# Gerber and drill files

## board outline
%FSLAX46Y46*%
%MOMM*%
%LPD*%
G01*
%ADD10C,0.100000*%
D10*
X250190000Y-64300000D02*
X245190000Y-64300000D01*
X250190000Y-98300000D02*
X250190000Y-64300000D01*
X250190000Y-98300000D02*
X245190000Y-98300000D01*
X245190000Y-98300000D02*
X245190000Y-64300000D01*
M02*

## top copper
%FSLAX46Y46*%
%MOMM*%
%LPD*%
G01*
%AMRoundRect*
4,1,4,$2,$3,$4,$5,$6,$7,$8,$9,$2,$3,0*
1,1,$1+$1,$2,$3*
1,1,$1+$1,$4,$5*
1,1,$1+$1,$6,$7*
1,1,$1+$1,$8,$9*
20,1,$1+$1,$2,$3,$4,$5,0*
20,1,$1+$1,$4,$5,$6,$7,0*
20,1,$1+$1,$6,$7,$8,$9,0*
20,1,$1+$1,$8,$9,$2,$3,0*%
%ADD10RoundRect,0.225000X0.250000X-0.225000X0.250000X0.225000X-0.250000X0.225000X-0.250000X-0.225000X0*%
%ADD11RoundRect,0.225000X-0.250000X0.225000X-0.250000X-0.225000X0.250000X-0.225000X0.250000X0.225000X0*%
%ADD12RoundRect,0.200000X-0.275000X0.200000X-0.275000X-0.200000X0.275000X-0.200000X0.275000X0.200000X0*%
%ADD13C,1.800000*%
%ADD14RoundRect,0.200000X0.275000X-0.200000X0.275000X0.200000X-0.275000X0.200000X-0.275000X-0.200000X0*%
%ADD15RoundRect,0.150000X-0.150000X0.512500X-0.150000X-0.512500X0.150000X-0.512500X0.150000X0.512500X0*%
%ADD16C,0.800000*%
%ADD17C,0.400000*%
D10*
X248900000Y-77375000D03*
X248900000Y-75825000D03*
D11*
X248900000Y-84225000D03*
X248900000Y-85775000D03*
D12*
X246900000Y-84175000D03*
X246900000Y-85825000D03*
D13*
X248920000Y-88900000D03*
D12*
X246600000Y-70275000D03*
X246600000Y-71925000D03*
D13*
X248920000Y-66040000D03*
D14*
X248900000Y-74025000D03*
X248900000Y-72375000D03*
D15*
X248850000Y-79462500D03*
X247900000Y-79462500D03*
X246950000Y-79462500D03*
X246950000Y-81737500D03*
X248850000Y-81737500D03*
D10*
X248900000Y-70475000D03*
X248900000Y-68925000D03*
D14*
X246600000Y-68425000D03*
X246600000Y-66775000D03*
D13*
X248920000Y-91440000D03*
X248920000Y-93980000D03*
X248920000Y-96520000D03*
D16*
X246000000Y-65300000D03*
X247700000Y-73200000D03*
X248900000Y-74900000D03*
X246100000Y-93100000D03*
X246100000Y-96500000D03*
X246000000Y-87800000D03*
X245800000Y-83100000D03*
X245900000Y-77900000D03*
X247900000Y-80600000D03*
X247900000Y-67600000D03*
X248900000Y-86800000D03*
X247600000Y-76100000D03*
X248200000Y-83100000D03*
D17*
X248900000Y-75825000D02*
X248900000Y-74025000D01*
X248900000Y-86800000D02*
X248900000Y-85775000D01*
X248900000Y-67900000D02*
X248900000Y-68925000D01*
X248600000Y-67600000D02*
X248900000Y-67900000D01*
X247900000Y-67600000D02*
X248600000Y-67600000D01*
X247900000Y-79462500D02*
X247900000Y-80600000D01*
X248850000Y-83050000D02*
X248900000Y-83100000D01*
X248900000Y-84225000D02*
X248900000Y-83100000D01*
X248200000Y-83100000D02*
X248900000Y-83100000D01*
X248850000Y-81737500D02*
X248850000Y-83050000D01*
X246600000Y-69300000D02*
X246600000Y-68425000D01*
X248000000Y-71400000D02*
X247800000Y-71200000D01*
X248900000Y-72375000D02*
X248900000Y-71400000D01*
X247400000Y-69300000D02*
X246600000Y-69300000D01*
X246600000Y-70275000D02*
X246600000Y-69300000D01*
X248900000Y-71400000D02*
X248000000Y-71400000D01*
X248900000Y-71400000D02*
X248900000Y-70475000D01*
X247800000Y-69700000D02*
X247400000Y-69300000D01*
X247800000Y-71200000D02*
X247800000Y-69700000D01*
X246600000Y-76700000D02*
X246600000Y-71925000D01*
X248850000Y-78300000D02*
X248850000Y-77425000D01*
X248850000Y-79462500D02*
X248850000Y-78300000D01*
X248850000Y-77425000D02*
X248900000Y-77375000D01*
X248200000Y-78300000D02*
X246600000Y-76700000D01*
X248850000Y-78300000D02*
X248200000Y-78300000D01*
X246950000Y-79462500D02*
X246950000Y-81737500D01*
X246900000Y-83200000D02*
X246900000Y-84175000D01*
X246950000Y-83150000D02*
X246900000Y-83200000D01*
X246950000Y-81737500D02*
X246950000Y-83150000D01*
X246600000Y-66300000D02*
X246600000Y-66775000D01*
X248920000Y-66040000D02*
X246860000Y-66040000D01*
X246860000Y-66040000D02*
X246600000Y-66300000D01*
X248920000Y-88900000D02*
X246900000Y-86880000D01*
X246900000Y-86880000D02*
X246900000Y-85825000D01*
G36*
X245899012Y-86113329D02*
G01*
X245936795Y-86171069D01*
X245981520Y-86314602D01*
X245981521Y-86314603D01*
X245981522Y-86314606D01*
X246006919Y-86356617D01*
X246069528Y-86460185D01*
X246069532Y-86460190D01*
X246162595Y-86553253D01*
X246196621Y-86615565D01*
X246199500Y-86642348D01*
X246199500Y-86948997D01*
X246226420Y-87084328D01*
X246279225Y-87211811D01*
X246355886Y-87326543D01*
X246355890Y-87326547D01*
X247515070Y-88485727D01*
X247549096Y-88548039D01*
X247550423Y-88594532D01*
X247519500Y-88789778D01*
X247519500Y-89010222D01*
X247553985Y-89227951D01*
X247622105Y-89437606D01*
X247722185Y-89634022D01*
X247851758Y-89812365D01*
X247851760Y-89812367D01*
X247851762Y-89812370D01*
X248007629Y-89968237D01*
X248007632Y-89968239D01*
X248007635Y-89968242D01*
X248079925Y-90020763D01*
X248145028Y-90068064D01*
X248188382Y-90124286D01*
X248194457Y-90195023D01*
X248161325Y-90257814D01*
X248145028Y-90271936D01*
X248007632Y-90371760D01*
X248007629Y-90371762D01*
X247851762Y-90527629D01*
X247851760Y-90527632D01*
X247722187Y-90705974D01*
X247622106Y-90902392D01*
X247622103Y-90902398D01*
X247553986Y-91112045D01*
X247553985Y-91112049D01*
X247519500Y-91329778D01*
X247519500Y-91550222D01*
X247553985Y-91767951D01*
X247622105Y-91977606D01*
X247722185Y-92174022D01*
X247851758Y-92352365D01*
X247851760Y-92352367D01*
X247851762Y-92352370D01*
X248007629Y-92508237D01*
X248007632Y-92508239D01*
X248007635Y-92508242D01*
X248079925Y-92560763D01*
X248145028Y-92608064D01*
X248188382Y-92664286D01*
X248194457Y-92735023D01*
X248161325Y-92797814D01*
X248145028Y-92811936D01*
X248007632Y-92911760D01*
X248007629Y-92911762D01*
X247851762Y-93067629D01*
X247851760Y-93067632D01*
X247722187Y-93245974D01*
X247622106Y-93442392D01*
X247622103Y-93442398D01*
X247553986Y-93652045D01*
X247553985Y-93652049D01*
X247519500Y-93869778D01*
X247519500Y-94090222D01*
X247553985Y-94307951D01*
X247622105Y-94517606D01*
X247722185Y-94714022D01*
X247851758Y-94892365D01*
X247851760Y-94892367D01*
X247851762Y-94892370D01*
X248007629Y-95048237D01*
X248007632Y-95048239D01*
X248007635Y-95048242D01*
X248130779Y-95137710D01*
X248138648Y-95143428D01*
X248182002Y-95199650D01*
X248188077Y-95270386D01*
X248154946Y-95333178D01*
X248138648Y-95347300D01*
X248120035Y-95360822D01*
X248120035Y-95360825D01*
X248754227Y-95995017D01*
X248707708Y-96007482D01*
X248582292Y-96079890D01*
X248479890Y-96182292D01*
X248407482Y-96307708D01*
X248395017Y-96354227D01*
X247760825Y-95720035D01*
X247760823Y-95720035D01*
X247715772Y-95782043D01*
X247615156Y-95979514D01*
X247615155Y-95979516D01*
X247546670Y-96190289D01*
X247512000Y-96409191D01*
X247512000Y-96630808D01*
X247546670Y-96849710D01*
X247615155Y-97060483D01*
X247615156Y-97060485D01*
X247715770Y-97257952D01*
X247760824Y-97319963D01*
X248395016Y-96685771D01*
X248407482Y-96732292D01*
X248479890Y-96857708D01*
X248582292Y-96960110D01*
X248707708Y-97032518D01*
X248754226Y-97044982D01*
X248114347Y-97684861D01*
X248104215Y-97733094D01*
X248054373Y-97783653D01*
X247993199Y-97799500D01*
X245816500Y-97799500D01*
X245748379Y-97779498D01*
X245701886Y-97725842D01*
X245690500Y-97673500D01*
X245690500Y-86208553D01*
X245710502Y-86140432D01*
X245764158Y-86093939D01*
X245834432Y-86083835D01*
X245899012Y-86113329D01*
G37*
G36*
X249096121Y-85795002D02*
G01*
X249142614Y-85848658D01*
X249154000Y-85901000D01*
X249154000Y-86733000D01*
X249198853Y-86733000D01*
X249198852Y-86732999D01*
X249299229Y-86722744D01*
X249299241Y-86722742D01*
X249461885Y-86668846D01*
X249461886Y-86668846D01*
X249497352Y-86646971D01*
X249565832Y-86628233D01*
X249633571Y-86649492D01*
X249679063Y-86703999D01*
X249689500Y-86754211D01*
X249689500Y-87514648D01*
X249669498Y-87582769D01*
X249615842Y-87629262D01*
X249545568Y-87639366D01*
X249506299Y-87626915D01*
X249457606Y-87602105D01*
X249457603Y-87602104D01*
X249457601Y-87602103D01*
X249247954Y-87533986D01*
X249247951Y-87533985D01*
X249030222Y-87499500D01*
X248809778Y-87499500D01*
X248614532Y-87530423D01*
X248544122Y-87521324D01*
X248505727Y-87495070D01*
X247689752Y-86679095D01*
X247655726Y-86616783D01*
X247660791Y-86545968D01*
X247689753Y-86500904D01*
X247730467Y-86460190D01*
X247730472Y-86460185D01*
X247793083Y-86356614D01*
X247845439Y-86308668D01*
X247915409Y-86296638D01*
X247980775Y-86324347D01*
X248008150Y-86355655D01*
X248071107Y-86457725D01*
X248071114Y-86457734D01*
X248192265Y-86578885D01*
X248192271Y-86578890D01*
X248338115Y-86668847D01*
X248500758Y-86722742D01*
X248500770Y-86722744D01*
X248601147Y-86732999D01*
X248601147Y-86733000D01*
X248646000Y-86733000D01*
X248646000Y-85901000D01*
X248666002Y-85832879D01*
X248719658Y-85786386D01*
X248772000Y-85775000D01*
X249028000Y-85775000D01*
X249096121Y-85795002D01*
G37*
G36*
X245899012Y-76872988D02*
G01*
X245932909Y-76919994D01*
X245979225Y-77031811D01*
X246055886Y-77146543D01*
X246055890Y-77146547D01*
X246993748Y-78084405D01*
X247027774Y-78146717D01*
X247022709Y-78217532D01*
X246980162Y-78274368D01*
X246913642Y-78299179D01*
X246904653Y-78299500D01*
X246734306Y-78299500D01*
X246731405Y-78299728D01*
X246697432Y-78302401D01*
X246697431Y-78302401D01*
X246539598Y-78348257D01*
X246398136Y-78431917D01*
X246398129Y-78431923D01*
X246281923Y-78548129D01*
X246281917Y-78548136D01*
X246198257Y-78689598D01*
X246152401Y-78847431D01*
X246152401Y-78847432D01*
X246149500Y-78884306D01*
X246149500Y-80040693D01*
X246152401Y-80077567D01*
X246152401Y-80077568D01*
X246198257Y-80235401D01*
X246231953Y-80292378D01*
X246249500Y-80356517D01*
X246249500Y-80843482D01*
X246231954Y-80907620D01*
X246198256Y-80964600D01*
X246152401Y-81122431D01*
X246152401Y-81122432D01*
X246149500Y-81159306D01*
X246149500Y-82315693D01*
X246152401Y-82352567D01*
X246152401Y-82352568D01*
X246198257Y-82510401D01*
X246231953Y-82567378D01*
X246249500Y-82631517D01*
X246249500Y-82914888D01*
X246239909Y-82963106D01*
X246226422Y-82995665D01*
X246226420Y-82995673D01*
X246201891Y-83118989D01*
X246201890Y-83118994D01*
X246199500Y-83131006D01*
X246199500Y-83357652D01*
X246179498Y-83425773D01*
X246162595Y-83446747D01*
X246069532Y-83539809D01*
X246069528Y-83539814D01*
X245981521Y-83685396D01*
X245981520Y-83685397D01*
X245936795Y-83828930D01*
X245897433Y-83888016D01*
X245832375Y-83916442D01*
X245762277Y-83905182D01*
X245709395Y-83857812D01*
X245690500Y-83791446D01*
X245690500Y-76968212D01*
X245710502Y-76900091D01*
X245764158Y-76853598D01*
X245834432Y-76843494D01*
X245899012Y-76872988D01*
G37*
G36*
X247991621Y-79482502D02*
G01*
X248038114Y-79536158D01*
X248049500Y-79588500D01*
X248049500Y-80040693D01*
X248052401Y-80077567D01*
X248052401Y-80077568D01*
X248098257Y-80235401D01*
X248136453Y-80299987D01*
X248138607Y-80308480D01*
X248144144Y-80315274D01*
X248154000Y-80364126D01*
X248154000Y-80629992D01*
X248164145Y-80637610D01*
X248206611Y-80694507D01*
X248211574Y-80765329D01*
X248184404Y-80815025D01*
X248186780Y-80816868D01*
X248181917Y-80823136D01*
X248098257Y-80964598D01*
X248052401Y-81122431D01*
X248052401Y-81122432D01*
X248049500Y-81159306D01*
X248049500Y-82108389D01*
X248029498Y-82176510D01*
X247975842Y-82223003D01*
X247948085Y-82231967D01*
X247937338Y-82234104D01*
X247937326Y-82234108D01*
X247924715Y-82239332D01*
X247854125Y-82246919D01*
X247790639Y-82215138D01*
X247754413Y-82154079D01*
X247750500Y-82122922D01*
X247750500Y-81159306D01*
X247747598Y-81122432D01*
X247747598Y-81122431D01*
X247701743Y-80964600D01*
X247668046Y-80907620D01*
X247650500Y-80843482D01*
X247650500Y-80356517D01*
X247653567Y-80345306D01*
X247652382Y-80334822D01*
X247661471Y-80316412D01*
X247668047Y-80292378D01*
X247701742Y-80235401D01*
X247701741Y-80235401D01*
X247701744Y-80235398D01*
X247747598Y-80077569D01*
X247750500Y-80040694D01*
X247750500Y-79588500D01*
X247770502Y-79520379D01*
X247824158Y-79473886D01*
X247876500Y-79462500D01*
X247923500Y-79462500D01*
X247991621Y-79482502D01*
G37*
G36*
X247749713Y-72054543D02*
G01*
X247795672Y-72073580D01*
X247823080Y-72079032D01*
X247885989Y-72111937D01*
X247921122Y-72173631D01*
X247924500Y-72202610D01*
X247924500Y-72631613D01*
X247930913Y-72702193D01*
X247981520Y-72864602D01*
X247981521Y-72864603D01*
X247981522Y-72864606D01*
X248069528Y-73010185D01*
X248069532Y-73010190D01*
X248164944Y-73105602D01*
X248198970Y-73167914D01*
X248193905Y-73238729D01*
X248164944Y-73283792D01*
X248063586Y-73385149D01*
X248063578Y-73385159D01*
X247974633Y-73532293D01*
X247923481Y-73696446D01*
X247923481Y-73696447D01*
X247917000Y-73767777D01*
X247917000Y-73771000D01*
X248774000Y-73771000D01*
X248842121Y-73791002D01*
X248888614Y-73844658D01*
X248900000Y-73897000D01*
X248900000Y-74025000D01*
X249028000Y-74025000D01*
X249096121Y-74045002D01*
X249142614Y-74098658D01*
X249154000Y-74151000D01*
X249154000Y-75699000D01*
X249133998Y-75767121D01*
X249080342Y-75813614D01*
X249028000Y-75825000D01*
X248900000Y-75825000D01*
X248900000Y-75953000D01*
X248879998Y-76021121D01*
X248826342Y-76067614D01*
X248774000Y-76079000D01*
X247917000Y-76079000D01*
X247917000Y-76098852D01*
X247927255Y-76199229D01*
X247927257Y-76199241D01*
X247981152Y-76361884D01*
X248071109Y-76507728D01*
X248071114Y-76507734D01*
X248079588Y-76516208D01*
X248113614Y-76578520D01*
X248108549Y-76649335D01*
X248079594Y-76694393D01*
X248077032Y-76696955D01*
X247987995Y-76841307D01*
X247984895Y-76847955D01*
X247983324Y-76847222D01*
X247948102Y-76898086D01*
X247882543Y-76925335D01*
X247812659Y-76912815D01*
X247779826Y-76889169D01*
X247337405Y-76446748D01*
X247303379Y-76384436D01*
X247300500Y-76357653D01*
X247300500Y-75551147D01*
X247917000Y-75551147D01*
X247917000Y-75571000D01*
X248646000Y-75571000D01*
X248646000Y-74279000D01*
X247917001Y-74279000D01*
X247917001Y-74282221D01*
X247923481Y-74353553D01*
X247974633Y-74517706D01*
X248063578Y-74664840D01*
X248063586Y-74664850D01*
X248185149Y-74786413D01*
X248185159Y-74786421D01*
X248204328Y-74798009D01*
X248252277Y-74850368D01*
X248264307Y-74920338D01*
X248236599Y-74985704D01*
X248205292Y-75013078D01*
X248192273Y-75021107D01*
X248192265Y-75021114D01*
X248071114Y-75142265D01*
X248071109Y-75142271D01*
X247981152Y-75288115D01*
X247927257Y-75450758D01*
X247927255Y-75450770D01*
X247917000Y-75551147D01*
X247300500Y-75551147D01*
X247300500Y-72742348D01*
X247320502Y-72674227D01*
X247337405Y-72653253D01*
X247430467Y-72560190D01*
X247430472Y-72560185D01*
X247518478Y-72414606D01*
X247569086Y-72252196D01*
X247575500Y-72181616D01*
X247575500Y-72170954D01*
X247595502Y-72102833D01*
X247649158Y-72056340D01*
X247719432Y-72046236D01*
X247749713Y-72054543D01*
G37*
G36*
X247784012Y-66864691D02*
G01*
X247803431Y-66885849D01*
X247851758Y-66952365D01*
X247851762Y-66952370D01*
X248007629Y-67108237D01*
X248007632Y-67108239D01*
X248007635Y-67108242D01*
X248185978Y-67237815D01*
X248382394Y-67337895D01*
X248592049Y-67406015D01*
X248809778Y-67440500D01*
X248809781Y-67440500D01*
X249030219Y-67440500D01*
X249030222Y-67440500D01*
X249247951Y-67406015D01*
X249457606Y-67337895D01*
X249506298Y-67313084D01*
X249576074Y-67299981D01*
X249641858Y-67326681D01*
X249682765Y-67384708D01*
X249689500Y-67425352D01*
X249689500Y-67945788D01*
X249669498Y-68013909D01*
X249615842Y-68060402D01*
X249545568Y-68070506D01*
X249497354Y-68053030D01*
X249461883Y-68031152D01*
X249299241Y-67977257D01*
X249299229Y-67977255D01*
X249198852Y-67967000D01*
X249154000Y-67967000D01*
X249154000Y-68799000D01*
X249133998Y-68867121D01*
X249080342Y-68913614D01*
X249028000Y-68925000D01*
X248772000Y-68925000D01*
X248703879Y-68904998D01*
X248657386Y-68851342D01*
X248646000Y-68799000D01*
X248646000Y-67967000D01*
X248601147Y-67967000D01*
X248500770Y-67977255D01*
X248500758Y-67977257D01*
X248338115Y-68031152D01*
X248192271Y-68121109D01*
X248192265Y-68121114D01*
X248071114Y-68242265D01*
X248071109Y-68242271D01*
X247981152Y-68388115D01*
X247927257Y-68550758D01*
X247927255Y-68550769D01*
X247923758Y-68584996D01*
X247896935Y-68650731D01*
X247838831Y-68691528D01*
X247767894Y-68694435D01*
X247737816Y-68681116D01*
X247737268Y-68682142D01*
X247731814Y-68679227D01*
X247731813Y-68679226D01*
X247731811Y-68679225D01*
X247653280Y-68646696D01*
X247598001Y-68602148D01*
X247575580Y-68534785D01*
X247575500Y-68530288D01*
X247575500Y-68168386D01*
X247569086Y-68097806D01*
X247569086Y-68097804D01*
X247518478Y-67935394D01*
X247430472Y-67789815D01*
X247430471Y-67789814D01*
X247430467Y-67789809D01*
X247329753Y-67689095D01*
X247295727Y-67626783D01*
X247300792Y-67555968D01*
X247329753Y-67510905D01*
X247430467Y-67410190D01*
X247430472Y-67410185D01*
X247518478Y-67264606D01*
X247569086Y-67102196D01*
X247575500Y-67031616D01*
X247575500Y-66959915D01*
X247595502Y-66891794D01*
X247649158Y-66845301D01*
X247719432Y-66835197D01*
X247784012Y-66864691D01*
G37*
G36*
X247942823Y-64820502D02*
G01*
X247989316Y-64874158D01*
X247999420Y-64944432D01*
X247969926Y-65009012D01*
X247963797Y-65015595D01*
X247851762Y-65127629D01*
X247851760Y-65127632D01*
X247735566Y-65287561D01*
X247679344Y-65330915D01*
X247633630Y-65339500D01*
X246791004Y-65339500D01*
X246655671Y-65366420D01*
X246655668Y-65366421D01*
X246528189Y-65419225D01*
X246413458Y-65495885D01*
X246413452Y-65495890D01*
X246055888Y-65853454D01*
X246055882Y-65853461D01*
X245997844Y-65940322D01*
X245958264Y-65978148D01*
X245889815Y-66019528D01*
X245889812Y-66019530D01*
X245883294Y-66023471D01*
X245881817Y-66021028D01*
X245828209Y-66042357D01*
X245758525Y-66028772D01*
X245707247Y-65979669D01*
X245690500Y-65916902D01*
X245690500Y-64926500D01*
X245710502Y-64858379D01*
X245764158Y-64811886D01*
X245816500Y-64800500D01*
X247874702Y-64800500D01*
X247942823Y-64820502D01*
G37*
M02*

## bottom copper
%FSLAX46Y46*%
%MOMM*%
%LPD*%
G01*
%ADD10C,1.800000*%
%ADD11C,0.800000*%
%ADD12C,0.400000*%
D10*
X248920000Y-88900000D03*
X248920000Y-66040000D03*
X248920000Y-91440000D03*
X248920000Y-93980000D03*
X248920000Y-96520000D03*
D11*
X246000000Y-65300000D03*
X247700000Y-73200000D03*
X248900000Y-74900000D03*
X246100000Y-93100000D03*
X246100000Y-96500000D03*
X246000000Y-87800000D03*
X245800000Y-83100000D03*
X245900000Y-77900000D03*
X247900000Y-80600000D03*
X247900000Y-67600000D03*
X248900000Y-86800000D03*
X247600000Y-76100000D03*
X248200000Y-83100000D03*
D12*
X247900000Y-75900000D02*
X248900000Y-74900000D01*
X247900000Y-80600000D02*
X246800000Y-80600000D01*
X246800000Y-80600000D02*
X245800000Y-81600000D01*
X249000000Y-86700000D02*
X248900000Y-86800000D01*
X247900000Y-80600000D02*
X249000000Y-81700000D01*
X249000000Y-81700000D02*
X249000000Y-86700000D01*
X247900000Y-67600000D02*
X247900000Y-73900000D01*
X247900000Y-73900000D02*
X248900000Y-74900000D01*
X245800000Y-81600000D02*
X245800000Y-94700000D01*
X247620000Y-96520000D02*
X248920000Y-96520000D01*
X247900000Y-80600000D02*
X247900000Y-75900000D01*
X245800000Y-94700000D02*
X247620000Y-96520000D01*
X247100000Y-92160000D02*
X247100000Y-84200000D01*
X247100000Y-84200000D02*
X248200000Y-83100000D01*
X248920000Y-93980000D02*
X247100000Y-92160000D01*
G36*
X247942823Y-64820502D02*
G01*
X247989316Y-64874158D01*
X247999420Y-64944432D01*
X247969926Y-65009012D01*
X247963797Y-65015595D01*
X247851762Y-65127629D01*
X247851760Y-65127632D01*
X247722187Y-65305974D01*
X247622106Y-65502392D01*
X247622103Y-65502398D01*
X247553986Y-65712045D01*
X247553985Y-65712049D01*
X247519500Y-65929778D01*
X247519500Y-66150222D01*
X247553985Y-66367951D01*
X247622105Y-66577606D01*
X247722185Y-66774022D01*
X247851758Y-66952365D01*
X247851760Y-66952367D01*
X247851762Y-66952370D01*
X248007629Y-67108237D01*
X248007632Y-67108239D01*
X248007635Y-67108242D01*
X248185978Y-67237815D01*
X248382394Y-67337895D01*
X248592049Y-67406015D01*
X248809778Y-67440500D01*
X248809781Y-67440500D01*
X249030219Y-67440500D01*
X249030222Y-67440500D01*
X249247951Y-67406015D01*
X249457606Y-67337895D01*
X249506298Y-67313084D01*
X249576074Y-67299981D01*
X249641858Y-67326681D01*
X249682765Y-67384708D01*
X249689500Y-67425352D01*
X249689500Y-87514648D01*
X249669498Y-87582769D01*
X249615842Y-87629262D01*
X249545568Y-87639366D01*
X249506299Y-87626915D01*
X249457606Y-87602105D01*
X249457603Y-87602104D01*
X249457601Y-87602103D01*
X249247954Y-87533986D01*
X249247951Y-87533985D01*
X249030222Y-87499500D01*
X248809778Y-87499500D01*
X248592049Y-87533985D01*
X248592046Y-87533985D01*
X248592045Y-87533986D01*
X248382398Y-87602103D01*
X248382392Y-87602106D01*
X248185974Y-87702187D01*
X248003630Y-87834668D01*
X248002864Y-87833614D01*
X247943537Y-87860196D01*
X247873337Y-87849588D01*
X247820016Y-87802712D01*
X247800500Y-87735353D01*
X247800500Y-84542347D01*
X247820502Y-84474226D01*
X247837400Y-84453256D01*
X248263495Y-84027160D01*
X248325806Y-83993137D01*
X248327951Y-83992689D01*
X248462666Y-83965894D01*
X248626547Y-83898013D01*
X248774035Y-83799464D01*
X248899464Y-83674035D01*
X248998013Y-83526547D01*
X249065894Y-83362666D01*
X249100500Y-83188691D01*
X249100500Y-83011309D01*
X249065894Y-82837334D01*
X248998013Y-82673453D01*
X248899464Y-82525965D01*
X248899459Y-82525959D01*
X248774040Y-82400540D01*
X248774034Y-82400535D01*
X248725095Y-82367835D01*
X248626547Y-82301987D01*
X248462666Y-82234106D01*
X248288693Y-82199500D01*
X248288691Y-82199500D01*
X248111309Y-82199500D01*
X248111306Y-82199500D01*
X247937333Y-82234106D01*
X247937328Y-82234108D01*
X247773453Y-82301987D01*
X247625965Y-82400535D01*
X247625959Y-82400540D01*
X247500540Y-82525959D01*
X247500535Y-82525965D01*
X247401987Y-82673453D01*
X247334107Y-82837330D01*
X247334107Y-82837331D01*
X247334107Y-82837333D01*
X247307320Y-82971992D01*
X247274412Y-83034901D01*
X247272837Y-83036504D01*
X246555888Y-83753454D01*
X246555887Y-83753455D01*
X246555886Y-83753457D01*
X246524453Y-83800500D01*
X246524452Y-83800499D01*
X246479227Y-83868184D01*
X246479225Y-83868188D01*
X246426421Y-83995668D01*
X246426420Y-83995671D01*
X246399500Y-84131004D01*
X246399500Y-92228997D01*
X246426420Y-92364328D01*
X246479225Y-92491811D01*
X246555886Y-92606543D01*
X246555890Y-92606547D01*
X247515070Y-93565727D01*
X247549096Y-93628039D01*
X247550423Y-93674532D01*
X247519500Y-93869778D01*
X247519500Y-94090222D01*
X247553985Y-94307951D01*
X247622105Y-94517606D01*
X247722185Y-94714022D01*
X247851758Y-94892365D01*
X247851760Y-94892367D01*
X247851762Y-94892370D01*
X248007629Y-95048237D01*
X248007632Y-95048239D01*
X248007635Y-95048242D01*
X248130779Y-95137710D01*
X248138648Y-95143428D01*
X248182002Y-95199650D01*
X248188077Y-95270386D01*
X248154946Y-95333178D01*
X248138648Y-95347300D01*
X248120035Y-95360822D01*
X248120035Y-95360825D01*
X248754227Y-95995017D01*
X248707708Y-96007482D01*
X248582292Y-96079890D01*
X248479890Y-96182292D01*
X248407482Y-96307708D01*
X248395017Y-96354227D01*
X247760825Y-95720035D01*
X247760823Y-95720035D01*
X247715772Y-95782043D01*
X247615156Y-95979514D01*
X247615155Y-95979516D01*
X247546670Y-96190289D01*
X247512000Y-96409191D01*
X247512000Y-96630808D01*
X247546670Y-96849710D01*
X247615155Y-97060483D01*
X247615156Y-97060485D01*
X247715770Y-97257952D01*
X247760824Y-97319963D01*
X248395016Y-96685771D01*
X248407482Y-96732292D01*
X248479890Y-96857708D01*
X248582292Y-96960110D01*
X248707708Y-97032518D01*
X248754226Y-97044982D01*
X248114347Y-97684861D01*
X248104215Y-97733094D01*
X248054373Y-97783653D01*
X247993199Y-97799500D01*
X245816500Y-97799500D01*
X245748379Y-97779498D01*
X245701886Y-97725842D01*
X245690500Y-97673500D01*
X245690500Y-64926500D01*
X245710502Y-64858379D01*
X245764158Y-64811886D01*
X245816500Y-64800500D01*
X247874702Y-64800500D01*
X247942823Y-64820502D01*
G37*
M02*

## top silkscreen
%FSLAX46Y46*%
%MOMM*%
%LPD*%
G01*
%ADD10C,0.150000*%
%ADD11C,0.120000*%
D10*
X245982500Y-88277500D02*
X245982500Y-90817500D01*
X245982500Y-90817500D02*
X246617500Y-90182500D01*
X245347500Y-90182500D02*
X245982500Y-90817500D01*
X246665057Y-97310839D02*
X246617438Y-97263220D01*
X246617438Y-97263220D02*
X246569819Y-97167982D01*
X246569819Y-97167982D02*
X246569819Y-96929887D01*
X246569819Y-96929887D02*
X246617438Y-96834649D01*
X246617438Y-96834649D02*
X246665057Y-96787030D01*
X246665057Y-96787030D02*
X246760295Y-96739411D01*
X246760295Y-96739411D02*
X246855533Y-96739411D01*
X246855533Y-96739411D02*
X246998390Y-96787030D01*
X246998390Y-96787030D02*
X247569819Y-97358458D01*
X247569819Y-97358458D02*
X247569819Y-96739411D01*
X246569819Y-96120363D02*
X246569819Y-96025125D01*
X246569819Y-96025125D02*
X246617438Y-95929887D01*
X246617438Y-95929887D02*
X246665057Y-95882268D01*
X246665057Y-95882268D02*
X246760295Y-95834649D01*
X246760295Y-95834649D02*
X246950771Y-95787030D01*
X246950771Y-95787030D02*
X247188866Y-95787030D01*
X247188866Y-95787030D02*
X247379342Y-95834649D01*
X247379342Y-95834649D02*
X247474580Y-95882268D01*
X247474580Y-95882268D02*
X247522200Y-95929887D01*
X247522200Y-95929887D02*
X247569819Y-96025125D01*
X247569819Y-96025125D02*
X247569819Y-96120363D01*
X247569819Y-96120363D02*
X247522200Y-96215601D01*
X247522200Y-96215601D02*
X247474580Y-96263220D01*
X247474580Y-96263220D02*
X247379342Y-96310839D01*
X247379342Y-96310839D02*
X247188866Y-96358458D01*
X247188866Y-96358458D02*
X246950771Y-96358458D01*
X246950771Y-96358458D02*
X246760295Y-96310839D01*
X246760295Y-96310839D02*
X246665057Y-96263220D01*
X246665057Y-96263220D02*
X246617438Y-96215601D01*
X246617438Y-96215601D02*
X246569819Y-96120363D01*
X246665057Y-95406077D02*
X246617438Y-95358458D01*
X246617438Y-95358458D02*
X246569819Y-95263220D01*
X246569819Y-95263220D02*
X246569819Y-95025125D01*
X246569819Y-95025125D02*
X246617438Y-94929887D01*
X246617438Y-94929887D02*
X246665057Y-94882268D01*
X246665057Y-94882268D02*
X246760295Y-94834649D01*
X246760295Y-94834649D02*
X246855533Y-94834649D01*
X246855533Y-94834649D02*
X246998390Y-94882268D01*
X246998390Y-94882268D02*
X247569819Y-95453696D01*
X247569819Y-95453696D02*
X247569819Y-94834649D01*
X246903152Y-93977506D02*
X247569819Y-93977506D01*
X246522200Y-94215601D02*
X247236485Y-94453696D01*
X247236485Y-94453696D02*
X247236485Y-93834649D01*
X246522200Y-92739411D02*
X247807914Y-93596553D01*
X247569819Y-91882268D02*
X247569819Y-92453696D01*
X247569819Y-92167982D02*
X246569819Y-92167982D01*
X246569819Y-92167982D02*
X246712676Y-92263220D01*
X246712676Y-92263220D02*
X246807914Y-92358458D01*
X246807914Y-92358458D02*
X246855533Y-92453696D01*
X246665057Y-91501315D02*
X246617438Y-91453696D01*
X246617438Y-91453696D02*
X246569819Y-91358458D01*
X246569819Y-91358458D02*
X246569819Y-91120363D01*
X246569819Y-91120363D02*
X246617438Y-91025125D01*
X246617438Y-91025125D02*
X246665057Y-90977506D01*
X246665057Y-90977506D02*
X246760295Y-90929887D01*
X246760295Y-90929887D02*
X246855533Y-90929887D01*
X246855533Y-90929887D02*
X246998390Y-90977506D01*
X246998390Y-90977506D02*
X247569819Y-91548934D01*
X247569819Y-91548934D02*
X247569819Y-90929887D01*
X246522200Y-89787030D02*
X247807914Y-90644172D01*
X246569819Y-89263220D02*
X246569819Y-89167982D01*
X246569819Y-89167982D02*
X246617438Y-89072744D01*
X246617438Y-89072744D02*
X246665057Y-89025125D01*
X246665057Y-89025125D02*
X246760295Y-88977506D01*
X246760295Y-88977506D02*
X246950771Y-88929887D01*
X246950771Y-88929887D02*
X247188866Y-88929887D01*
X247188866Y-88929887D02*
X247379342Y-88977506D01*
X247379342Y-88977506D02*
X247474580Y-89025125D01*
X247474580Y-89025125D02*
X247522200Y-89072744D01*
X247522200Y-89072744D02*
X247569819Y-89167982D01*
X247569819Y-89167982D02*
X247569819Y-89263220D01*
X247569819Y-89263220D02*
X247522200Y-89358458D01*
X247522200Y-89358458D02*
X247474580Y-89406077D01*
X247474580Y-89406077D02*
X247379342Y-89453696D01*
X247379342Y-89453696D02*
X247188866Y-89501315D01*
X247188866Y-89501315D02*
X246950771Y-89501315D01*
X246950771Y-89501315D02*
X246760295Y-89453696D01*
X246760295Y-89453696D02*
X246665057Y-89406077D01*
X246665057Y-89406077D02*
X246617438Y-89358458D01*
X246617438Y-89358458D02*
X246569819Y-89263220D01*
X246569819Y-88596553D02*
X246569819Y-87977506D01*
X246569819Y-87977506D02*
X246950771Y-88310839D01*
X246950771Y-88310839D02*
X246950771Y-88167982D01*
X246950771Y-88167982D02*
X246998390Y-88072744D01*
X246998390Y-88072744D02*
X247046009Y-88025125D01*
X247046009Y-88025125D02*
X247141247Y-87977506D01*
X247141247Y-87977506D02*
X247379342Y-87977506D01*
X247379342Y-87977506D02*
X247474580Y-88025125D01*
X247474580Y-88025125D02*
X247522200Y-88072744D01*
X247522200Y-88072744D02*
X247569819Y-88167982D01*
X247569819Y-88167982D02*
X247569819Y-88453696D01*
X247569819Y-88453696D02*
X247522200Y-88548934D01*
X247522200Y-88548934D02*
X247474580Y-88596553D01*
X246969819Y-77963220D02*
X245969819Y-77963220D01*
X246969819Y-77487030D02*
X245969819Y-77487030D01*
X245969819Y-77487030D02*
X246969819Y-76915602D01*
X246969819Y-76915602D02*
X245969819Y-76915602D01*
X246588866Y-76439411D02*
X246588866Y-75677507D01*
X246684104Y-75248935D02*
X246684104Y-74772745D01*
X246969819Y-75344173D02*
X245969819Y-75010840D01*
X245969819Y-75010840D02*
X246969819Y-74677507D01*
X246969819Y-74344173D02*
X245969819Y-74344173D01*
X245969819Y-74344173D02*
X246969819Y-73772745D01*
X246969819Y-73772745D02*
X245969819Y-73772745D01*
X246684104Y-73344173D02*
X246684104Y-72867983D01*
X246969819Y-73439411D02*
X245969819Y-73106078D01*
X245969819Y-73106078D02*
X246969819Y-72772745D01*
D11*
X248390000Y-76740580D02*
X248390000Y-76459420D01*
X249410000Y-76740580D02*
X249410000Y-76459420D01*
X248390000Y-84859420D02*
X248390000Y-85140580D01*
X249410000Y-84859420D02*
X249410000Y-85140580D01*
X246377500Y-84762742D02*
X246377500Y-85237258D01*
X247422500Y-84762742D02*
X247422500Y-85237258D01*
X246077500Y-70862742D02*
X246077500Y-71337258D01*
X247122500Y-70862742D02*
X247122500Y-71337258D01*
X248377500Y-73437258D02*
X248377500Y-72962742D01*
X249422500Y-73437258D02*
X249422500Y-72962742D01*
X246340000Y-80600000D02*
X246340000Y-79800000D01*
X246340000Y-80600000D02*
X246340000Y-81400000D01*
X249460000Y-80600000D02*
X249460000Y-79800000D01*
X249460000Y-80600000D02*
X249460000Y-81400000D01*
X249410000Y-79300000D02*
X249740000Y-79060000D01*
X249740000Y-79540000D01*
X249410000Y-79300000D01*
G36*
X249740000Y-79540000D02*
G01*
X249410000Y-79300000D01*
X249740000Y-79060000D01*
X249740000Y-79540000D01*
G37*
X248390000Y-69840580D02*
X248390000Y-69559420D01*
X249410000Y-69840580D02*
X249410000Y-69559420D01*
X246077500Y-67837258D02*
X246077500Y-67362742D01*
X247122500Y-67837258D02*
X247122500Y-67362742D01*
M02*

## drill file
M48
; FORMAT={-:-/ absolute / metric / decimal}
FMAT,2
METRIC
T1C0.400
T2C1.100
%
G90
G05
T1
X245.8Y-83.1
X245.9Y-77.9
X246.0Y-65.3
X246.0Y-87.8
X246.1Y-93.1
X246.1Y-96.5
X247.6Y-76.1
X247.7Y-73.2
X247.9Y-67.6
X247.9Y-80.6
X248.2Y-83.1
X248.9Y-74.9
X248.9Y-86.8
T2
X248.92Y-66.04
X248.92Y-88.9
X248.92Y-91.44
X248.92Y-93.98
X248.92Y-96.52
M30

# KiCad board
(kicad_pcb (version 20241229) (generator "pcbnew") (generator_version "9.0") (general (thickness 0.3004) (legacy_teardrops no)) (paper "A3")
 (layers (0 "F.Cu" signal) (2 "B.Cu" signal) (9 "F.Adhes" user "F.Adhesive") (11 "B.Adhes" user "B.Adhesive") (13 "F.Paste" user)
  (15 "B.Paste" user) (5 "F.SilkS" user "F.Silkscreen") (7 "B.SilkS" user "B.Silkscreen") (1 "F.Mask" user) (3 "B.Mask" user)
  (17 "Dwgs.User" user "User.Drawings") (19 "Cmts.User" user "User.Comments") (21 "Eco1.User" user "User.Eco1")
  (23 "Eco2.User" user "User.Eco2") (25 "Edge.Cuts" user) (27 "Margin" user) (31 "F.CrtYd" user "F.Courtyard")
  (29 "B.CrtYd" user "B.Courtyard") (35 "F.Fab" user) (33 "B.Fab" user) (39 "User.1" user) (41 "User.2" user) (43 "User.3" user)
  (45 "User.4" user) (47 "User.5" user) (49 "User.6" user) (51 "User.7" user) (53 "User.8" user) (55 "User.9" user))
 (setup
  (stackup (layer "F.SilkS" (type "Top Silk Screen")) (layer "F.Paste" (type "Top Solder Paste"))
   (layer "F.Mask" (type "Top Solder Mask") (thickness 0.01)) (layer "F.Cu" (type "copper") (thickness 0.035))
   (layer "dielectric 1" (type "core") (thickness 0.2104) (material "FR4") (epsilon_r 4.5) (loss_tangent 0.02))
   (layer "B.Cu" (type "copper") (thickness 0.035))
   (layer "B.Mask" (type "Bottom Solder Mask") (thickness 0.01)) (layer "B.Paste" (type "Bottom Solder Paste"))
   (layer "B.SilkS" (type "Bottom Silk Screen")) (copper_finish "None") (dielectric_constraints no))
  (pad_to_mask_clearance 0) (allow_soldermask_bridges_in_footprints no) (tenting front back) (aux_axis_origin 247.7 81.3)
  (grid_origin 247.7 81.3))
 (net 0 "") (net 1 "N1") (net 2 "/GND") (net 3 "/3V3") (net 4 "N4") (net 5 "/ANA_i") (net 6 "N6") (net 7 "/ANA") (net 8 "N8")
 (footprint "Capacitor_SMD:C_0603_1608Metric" (layer "F.Cu") (at 248.9 76.6 90)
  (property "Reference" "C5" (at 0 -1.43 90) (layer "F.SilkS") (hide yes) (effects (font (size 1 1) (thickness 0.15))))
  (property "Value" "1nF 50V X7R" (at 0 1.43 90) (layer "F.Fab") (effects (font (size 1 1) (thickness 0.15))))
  (fp_line (start -0.14058 -0.51) (end 0.14058 -0.51) (stroke (width 0.12) (type solid)) (layer "F.SilkS"))
  (fp_line (start -0.14058 0.51) (end 0.14058 0.51) (stroke (width 0.12) (type solid)) (layer "F.SilkS"))
  (pad "1" smd roundrect (at -0.775 0 90) (size 0.9 0.95) (layers "F.Cu" "F.Mask" "F.Paste") (roundrect_rratio 0.25) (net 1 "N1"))
  (pad "2" smd roundrect (at 0.775 0 90) (size 0.9 0.95) (layers "F.Cu" "F.Mask" "F.Paste") (roundrect_rratio 0.25) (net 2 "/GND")))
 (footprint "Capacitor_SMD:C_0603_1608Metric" (layer "F.Cu") (at 248.9 85 -90)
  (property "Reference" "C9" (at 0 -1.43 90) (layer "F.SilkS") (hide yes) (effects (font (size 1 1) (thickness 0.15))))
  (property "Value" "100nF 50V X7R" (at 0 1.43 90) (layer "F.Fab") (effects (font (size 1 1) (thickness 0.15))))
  (fp_line (start -0.14058 0.51) (end 0.14058 0.51) (stroke (width 0.12) (type solid)) (layer "F.SilkS"))
  (fp_line (start -0.14058 -0.51) (end 0.14058 -0.51) (stroke (width 0.12) (type solid)) (layer "F.SilkS"))
  (pad "1" smd roundrect (at -0.775 0 270) (size 0.9 0.95) (layers "F.Cu" "F.Mask" "F.Paste") (roundrect_rratio 0.25) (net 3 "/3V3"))
  (pad "2" smd roundrect (at 0.775 0 270) (size 0.9 0.95) (layers "F.Cu" "F.Mask" "F.Paste") (roundrect_rratio 0.25) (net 2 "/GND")))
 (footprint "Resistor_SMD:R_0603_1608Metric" (layer "F.Cu") (at 246.9 85 -90)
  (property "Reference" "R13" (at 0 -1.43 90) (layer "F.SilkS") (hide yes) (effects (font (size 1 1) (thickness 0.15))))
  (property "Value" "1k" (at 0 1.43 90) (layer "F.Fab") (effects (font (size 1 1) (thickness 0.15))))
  (fp_line (start -0.237258 0.5225) (end 0.237258 0.5225) (stroke (width 0.12) (type solid)) (layer "F.SilkS"))
  (fp_line (start -0.237258 -0.5225) (end 0.237258 -0.5225) (stroke (width 0.12) (type solid)) (layer "F.SilkS"))
  (pad "1" smd roundrect (at -0.825 0 270) (size 0.8 0.95) (layers "F.Cu" "F.Mask" "F.Paste") (roundrect_rratio 0.25) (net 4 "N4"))
  (pad "2" smd roundrect (at 0.825 0 270) (size 0.8 0.95) (layers "F.Cu" "F.Mask" "F.Paste") (roundrect_rratio 0.25) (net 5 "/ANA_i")))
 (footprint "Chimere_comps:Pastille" (layer "F.Cu") (at 248.92 88.9)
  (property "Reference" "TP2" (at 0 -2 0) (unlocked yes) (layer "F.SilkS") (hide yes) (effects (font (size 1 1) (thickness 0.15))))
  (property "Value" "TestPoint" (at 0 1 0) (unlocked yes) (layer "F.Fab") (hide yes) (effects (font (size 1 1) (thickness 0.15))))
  (pad "1" thru_hole circle (at 0 0) (size 1.8 1.8) (drill 1.1) (layers "*.Cu" "*.Mask") (remove_unused_layers no) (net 5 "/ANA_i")))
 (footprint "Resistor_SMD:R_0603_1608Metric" (layer "F.Cu") (at 246.6 71.1 -90)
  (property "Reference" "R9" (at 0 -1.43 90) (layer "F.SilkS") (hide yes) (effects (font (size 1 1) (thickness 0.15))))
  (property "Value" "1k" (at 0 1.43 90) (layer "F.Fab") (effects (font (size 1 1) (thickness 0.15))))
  (fp_line (start -0.237258 0.5225) (end 0.237258 0.5225) (stroke (width 0.12) (type solid)) (layer "F.SilkS"))
  (fp_line (start -0.237258 -0.5225) (end 0.237258 -0.5225) (stroke (width 0.12) (type solid)) (layer "F.SilkS"))
  (pad "1" smd roundrect (at -0.825 0 270) (size 0.8 0.95) (layers "F.Cu" "F.Mask" "F.Paste") (roundrect_rratio 0.25) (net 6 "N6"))
  (pad "2" smd roundrect (at 0.825 0 270) (size 0.8 0.95) (layers "F.Cu" "F.Mask" "F.Paste") (roundrect_rratio 0.25) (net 1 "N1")))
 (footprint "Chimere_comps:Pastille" (layer "F.Cu") (at 248.92 66.04)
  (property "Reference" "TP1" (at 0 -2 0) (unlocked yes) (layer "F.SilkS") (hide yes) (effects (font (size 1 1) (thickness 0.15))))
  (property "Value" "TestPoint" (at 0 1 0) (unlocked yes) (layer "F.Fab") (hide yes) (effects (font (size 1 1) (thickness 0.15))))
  (pad "1" thru_hole circle (at 0 0) (size 1.8 1.8) (drill 1.1) (layers "*.Cu" "*.Mask") (remove_unused_layers no) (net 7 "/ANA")))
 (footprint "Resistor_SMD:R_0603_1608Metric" (layer "F.Cu") (at 248.9 73.2 90)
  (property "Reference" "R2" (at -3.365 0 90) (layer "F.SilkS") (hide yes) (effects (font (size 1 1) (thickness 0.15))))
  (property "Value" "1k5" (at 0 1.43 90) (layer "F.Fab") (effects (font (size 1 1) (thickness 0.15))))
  (fp_line (start -0.237258 -0.5225) (end 0.237258 -0.5225) (stroke (width 0.12) (type solid)) (layer "F.SilkS"))
  (fp_line (start -0.237258 0.5225) (end 0.237258 0.5225) (stroke (width 0.12) (type solid)) (layer "F.SilkS"))
  (pad "1" smd roundrect (at -0.825 0 90) (size 0.8 0.95) (layers "F.Cu" "F.Mask" "F.Paste") (roundrect_rratio 0.25) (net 2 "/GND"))
  (pad "2" smd roundrect (at 0.825 0 90) (size 0.8 0.95) (layers "F.Cu" "F.Mask" "F.Paste") (roundrect_rratio 0.25) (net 6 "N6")))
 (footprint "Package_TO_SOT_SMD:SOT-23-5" (layer "F.Cu") (at 247.9 80.6 -90)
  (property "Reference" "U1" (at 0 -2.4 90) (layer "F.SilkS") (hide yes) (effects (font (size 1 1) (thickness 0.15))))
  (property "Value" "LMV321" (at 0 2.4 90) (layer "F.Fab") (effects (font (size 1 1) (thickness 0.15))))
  (fp_line (start 0 1.56) (end -0.8 1.56) (stroke (width 0.12) (type solid)) (layer "F.SilkS"))
  (fp_line (start 0 1.56) (end 0.8 1.56) (stroke (width 0.12) (type solid)) (layer "F.SilkS"))
  (fp_line (start 0 -1.56) (end -0.8 -1.56) (stroke (width 0.12) (type solid)) (layer "F.SilkS"))
  (fp_line (start 0 -1.56) (end 0.8 -1.56) (stroke (width 0.12) (type solid)) (layer "F.SilkS"))
  (fp_poly
   (pts (xy -1.3 -1.51) (xy -1.54 -1.84) (xy -1.06 -1.84) (xy -1.3 -1.51)) (stroke (width 0.12) (type solid)) (fill yes) (layer "F.SilkS"))
  (pad "1" smd roundrect (at -1.1375 -0.95 270) (size 1.325 0.6) (layers "F.Cu" "F.Mask" "F.Paste") (roundrect_rratio 0.25) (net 1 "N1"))
  (pad "2" smd roundrect (at -1.1375 0 270) (size 1.325 0.6) (layers "F.Cu" "F.Mask" "F.Paste") (roundrect_rratio 0.25) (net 2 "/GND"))
  (pad "3" smd roundrect (at -1.1375 0.95 270) (size 1.325 0.6) (layers "F.Cu" "F.Mask" "F.Paste") (roundrect_rratio 0.25) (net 4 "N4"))
  (pad "4" smd roundrect (at 1.1375 0.95 270) (size 1.325 0.6) (layers "F.Cu" "F.Mask" "F.Paste") (roundrect_rratio 0.25) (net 4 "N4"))
  (pad "5" smd roundrect (at 1.1375 -0.95 270) (size 1.325 0.6) (layers "F.Cu" "F.Mask" "F.Paste") (roundrect_rratio 0.25) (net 3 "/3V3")))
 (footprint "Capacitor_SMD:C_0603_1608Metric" (layer "F.Cu") (at 248.9 69.7 90)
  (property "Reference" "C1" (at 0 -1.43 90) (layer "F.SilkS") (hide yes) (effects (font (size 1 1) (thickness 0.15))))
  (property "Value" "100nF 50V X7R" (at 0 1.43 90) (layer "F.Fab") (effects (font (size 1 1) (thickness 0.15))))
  (fp_line (start -0.14058 -0.51) (end 0.14058 -0.51) (stroke (width 0.12) (type solid)) (layer "F.SilkS"))
  (fp_line (start -0.14058 0.51) (end 0.14058 0.51) (stroke (width 0.12) (type solid)) (layer "F.SilkS"))
  (pad "1" smd roundrect (at -0.775 0 90) (size 0.9 0.95) (layers "F.Cu" "F.Mask" "F.Paste") (roundrect_rratio 0.25) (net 6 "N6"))
  (pad "2" smd roundrect (at 0.775 0 90) (size 0.9 0.95) (layers "F.Cu" "F.Mask" "F.Paste") (roundrect_rratio 0.25) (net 2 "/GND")))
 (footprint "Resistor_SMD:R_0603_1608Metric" (layer "F.Cu") (at 246.6 67.6 90)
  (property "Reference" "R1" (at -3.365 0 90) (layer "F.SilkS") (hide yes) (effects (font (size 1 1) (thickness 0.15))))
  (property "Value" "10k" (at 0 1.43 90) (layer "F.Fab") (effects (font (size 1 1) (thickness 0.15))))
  (fp_line (start -0.237258 -0.5225) (end 0.237258 -0.5225) (stroke (width 0.12) (type solid)) (layer "F.SilkS"))
  (fp_line (start -0.237258 0.5225) (end 0.237258 0.5225) (stroke (width 0.12) (type solid)) (layer "F.SilkS"))
  (pad "1" smd roundrect (at -0.825 0 90) (size 0.8 0.95) (layers "F.Cu" "F.Mask" "F.Paste") (roundrect_rratio 0.25) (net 6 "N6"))
  (pad "2" smd roundrect (at 0.825 0 90) (size 0.8 0.95) (layers "F.Cu" "F.Mask" "F.Paste") (roundrect_rratio 0.25) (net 7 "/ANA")))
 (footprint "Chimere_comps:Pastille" (layer "F.Cu") (at 248.92 91.44)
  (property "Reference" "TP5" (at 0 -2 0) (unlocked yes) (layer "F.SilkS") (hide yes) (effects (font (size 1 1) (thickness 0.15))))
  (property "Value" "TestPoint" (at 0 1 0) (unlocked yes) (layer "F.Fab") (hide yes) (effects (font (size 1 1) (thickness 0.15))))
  (pad "1" thru_hole circle (at 0 0) (size 1.8 1.8) (drill 1.1) (layers "*.Cu" "*.Mask") (remove_unused_layers no) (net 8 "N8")))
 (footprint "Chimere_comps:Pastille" (layer "F.Cu") (at 248.92 93.98)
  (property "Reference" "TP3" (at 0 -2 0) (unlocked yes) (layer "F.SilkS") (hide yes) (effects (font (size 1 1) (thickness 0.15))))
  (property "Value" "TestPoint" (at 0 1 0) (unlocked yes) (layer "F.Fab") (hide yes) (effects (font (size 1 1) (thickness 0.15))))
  (pad "1" thru_hole circle (at 0 0) (size 1.8 1.8) (drill 1.1) (layers "*.Cu" "*.Mask") (remove_unused_layers no) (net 3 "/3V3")))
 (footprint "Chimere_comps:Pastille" (layer "F.Cu") (at 248.92 96.52)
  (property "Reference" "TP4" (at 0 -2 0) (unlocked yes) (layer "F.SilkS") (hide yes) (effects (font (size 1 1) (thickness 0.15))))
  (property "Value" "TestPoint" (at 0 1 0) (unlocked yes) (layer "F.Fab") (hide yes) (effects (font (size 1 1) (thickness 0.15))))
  (pad "1" thru_hole circle (at 0 0) (size 1.8 1.8) (drill 1.1) (layers "*.Cu" "*.Mask") (remove_unused_layers no) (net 2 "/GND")))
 (gr_line (start 245.9825 88.2775) (end 245.9825 90.8175) (stroke (width 0.15) (type solid)) (layer "F.SilkS"))
 (gr_line (start 245.9825 90.8175) (end 246.6175 90.1825) (stroke (width 0.15) (type solid)) (layer "F.SilkS"))
 (gr_line (start 245.3475 90.1825) (end 245.9825 90.8175) (stroke (width 0.15) (type solid)) (layer "F.SilkS"))
 (gr_line (start 250.19 64.3) (end 245.19 64.3) (stroke (width 0.1) (type default)) (layer "Edge.Cuts"))
 (gr_line (start 250.19 98.3) (end 250.19 64.3) (stroke (width 0.1) (type default)) (layer "Edge.Cuts"))
 (gr_line (start 250.19 98.3) (end 245.19 98.3) (stroke (width 0.1) (type default)) (layer "Edge.Cuts"))
 (gr_line (start 245.19 98.3) (end 245.19 64.3) (stroke (width 0.1) (type default)) (layer "Edge.Cuts"))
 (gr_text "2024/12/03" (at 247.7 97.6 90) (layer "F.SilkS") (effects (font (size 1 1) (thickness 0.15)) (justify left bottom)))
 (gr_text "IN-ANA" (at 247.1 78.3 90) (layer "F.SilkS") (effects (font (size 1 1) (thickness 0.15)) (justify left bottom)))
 (segment (start 248.9 75.825) (end 248.9 74.025) (width 0.4) (layer "F.Cu") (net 2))
 (segment (start 248.9 86.8) (end 248.9 85.775) (width 0.4) (layer "F.Cu") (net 2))
 (segment (start 248.9 67.9) (end 248.9 68.925) (width 0.4) (layer "F.Cu") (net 2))
 (segment (start 248.6 67.6) (end 248.9 67.9) (width 0.4) (layer "F.Cu") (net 2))
 (segment (start 247.9 67.6) (end 248.6 67.6) (width 0.4) (layer "F.Cu") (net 2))
 (segment (start 247.9 79.4625) (end 247.9 80.6) (width 0.4) (layer "F.Cu") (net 2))
 (via (at 246 65.3) (size 0.8) (drill 0.4) (layers "F.Cu" "B.Cu") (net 2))
 (via (at 247.7 73.2) (size 0.8) (drill 0.4) (layers "F.Cu" "B.Cu") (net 2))
 (via (at 248.9 74.9) (size 0.8) (drill 0.4) (layers "F.Cu" "B.Cu") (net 2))
 (via (at 246.1 93.1) (size 0.8) (drill 0.4) (layers "F.Cu" "B.Cu") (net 2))
 (via (at 246.1 96.5) (size 0.8) (drill 0.4) (layers "F.Cu" "B.Cu") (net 2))
 (via (at 246 87.8) (size 0.8) (drill 0.4) (layers "F.Cu" "B.Cu") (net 2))
 (via (at 245.8 83.1) (size 0.8) (drill 0.4) (layers "F.Cu" "B.Cu") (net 2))
 (via (at 245.9 77.9) (size 0.8) (drill 0.4) (layers "F.Cu" "B.Cu") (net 2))
 (via (at 247.9 80.6) (size 0.8) (drill 0.4) (layers "F.Cu" "B.Cu") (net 2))
 (via (at 247.9 67.6) (size 0.8) (drill 0.4) (layers "F.Cu" "B.Cu") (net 2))
 (via (at 248.9 86.8) (size 0.8) (drill 0.4) (layers "F.Cu" "B.Cu") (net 2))
 (via (at 247.6 76.1) (size 0.8) (drill 0.4) (layers "F.Cu" "B.Cu") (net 2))
 (segment (start 247.9 75.9) (end 248.9 74.9) (width 0.4) (layer "B.Cu") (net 2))
 (segment (start 247.9 80.6) (end 246.8 80.6) (width 0.4) (layer "B.Cu") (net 2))
 (segment (start 246.8 80.6) (end 245.8 81.6) (width 0.4) (layer "B.Cu") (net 2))
 (segment (start 249 86.7) (end 248.9 86.8) (width 0.4) (layer "B.Cu") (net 2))
 (segment (start 247.9 80.6) (end 249 81.7) (width 0.4) (layer "B.Cu") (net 2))
 (segment (start 249 81.7) (end 249 86.7) (width 0.4) (layer "B.Cu") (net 2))
 (segment (start 247.9 67.6) (end 247.9 73.9) (width 0.4) (layer "B.Cu") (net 2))
 (segment (start 247.9 73.9) (end 248.9 74.9) (width 0.4) (layer "B.Cu") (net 2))
 (segment (start 245.8 81.6) (end 245.8 94.7) (width 0.4) (layer "B.Cu") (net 2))
 (segment (start 247.62 96.52) (end 248.92 96.52) (width 0.4) (layer "B.Cu") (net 2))
 (segment (start 247.9 80.6) (end 247.9 75.9) (width 0.4) (layer "B.Cu") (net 2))
 (segment (start 245.8 94.7) (end 247.62 96.52) (width 0.4) (layer "B.Cu") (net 2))
 (segment (start 248.85 83.05) (end 248.9 83.1) (width 0.4) (layer "F.Cu") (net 3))
 (segment (start 248.9 84.225) (end 248.9 83.1) (width 0.4) (layer "F.Cu") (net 3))
 (segment (start 248.2 83.1) (end 248.9 83.1) (width 0.4) (layer "F.Cu") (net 3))
 (segment (start 248.85 81.7375) (end 248.85 83.05) (width 0.4) (layer "F.Cu") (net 3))
 (via (at 248.2 83.1) (size 0.8) (drill 0.4) (layers "F.Cu" "B.Cu") (free yes) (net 3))
 (segment (start 247.1 92.16) (end 247.1 84.2) (width 0.4) (layer "B.Cu") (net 3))
 (segment (start 247.1 84.2) (end 248.2 83.1) (width 0.4) (layer "B.Cu") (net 3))
 (segment (start 248.92 93.98) (end 247.1 92.16) (width 0.4) (layer "B.Cu") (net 3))
 (segment (start 246.6 69.3) (end 246.6 68.425) (width 0.4) (layer "F.Cu") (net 6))
 (segment (start 248 71.4) (end 247.8 71.2) (width 0.4) (layer "F.Cu") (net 6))
 (segment (start 248.9 72.375) (end 248.9 71.4) (width 0.4) (layer "F.Cu") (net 6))
 (segment (start 247.4 69.3) (end 246.6 69.3) (width 0.4) (layer "F.Cu") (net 6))
 (segment (start 246.6 70.275) (end 246.6 69.3) (width 0.4) (layer "F.Cu") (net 6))
 (segment (start 248.9 71.4) (end 248 71.4) (width 0.4) (layer "F.Cu") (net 6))
 (segment (start 248.9 71.4) (end 248.9 70.475) (width 0.4) (layer "F.Cu") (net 6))
 (segment (start 247.8 69.7) (end 247.4 69.3) (width 0.4) (layer "F.Cu") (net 6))
 (segment (start 247.8 71.2) (end 247.8 69.7) (width 0.4) (layer "F.Cu") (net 6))
 (segment (start 246.6 76.7) (end 246.6 71.925) (width 0.4) (layer "F.Cu") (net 1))
 (segment (start 248.85 78.3) (end 248.85 77.425) (width 0.4) (layer "F.Cu") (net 1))
 (segment (start 248.85 79.4625) (end 248.85 78.3) (width 0.4) (layer "F.Cu") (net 1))
 (segment (start 248.85 77.425) (end 248.9 77.375) (width 0.4) (layer "F.Cu") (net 1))
 (segment (start 248.2 78.3) (end 246.6 76.7) (width 0.4) (layer "F.Cu") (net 1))
 (segment (start 248.85 78.3) (end 248.2 78.3) (width 0.4) (layer "F.Cu") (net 1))
 (segment (start 246.95 79.4625) (end 246.95 81.7375) (width 0.4) (layer "F.Cu") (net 4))
 (segment (start 246.9 83.2) (end 246.9 84.175) (width 0.4) (layer "F.Cu") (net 4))
 (segment (start 246.95 83.15) (end 246.9 83.2) (width 0.4) (layer "F.Cu") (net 4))
 (segment (start 246.95 81.7375) (end 246.95 83.15) (width 0.4) (layer "F.Cu") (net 4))
 (segment (start 246.6 66.3) (end 246.6 66.775) (width 0.4) (layer "F.Cu") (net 7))
 (segment (start 248.92 66.04) (end 246.86 66.04) (width 0.4) (layer "F.Cu") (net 7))
 (segment (start 246.86 66.04) (end 246.6 66.3) (width 0.4) (layer "F.Cu") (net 7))
 (segment (start 248.92 88.9) (end 246.9 86.88) (width 0.4) (layer "F.Cu") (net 5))
 (segment (start 246.9 86.88) (end 246.9 85.825) (width 0.4) (layer "F.Cu") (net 5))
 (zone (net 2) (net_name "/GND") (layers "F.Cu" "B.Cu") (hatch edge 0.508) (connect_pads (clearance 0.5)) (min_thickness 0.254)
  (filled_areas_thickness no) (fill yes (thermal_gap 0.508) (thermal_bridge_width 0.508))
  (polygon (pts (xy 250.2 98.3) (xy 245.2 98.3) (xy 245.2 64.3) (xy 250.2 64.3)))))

